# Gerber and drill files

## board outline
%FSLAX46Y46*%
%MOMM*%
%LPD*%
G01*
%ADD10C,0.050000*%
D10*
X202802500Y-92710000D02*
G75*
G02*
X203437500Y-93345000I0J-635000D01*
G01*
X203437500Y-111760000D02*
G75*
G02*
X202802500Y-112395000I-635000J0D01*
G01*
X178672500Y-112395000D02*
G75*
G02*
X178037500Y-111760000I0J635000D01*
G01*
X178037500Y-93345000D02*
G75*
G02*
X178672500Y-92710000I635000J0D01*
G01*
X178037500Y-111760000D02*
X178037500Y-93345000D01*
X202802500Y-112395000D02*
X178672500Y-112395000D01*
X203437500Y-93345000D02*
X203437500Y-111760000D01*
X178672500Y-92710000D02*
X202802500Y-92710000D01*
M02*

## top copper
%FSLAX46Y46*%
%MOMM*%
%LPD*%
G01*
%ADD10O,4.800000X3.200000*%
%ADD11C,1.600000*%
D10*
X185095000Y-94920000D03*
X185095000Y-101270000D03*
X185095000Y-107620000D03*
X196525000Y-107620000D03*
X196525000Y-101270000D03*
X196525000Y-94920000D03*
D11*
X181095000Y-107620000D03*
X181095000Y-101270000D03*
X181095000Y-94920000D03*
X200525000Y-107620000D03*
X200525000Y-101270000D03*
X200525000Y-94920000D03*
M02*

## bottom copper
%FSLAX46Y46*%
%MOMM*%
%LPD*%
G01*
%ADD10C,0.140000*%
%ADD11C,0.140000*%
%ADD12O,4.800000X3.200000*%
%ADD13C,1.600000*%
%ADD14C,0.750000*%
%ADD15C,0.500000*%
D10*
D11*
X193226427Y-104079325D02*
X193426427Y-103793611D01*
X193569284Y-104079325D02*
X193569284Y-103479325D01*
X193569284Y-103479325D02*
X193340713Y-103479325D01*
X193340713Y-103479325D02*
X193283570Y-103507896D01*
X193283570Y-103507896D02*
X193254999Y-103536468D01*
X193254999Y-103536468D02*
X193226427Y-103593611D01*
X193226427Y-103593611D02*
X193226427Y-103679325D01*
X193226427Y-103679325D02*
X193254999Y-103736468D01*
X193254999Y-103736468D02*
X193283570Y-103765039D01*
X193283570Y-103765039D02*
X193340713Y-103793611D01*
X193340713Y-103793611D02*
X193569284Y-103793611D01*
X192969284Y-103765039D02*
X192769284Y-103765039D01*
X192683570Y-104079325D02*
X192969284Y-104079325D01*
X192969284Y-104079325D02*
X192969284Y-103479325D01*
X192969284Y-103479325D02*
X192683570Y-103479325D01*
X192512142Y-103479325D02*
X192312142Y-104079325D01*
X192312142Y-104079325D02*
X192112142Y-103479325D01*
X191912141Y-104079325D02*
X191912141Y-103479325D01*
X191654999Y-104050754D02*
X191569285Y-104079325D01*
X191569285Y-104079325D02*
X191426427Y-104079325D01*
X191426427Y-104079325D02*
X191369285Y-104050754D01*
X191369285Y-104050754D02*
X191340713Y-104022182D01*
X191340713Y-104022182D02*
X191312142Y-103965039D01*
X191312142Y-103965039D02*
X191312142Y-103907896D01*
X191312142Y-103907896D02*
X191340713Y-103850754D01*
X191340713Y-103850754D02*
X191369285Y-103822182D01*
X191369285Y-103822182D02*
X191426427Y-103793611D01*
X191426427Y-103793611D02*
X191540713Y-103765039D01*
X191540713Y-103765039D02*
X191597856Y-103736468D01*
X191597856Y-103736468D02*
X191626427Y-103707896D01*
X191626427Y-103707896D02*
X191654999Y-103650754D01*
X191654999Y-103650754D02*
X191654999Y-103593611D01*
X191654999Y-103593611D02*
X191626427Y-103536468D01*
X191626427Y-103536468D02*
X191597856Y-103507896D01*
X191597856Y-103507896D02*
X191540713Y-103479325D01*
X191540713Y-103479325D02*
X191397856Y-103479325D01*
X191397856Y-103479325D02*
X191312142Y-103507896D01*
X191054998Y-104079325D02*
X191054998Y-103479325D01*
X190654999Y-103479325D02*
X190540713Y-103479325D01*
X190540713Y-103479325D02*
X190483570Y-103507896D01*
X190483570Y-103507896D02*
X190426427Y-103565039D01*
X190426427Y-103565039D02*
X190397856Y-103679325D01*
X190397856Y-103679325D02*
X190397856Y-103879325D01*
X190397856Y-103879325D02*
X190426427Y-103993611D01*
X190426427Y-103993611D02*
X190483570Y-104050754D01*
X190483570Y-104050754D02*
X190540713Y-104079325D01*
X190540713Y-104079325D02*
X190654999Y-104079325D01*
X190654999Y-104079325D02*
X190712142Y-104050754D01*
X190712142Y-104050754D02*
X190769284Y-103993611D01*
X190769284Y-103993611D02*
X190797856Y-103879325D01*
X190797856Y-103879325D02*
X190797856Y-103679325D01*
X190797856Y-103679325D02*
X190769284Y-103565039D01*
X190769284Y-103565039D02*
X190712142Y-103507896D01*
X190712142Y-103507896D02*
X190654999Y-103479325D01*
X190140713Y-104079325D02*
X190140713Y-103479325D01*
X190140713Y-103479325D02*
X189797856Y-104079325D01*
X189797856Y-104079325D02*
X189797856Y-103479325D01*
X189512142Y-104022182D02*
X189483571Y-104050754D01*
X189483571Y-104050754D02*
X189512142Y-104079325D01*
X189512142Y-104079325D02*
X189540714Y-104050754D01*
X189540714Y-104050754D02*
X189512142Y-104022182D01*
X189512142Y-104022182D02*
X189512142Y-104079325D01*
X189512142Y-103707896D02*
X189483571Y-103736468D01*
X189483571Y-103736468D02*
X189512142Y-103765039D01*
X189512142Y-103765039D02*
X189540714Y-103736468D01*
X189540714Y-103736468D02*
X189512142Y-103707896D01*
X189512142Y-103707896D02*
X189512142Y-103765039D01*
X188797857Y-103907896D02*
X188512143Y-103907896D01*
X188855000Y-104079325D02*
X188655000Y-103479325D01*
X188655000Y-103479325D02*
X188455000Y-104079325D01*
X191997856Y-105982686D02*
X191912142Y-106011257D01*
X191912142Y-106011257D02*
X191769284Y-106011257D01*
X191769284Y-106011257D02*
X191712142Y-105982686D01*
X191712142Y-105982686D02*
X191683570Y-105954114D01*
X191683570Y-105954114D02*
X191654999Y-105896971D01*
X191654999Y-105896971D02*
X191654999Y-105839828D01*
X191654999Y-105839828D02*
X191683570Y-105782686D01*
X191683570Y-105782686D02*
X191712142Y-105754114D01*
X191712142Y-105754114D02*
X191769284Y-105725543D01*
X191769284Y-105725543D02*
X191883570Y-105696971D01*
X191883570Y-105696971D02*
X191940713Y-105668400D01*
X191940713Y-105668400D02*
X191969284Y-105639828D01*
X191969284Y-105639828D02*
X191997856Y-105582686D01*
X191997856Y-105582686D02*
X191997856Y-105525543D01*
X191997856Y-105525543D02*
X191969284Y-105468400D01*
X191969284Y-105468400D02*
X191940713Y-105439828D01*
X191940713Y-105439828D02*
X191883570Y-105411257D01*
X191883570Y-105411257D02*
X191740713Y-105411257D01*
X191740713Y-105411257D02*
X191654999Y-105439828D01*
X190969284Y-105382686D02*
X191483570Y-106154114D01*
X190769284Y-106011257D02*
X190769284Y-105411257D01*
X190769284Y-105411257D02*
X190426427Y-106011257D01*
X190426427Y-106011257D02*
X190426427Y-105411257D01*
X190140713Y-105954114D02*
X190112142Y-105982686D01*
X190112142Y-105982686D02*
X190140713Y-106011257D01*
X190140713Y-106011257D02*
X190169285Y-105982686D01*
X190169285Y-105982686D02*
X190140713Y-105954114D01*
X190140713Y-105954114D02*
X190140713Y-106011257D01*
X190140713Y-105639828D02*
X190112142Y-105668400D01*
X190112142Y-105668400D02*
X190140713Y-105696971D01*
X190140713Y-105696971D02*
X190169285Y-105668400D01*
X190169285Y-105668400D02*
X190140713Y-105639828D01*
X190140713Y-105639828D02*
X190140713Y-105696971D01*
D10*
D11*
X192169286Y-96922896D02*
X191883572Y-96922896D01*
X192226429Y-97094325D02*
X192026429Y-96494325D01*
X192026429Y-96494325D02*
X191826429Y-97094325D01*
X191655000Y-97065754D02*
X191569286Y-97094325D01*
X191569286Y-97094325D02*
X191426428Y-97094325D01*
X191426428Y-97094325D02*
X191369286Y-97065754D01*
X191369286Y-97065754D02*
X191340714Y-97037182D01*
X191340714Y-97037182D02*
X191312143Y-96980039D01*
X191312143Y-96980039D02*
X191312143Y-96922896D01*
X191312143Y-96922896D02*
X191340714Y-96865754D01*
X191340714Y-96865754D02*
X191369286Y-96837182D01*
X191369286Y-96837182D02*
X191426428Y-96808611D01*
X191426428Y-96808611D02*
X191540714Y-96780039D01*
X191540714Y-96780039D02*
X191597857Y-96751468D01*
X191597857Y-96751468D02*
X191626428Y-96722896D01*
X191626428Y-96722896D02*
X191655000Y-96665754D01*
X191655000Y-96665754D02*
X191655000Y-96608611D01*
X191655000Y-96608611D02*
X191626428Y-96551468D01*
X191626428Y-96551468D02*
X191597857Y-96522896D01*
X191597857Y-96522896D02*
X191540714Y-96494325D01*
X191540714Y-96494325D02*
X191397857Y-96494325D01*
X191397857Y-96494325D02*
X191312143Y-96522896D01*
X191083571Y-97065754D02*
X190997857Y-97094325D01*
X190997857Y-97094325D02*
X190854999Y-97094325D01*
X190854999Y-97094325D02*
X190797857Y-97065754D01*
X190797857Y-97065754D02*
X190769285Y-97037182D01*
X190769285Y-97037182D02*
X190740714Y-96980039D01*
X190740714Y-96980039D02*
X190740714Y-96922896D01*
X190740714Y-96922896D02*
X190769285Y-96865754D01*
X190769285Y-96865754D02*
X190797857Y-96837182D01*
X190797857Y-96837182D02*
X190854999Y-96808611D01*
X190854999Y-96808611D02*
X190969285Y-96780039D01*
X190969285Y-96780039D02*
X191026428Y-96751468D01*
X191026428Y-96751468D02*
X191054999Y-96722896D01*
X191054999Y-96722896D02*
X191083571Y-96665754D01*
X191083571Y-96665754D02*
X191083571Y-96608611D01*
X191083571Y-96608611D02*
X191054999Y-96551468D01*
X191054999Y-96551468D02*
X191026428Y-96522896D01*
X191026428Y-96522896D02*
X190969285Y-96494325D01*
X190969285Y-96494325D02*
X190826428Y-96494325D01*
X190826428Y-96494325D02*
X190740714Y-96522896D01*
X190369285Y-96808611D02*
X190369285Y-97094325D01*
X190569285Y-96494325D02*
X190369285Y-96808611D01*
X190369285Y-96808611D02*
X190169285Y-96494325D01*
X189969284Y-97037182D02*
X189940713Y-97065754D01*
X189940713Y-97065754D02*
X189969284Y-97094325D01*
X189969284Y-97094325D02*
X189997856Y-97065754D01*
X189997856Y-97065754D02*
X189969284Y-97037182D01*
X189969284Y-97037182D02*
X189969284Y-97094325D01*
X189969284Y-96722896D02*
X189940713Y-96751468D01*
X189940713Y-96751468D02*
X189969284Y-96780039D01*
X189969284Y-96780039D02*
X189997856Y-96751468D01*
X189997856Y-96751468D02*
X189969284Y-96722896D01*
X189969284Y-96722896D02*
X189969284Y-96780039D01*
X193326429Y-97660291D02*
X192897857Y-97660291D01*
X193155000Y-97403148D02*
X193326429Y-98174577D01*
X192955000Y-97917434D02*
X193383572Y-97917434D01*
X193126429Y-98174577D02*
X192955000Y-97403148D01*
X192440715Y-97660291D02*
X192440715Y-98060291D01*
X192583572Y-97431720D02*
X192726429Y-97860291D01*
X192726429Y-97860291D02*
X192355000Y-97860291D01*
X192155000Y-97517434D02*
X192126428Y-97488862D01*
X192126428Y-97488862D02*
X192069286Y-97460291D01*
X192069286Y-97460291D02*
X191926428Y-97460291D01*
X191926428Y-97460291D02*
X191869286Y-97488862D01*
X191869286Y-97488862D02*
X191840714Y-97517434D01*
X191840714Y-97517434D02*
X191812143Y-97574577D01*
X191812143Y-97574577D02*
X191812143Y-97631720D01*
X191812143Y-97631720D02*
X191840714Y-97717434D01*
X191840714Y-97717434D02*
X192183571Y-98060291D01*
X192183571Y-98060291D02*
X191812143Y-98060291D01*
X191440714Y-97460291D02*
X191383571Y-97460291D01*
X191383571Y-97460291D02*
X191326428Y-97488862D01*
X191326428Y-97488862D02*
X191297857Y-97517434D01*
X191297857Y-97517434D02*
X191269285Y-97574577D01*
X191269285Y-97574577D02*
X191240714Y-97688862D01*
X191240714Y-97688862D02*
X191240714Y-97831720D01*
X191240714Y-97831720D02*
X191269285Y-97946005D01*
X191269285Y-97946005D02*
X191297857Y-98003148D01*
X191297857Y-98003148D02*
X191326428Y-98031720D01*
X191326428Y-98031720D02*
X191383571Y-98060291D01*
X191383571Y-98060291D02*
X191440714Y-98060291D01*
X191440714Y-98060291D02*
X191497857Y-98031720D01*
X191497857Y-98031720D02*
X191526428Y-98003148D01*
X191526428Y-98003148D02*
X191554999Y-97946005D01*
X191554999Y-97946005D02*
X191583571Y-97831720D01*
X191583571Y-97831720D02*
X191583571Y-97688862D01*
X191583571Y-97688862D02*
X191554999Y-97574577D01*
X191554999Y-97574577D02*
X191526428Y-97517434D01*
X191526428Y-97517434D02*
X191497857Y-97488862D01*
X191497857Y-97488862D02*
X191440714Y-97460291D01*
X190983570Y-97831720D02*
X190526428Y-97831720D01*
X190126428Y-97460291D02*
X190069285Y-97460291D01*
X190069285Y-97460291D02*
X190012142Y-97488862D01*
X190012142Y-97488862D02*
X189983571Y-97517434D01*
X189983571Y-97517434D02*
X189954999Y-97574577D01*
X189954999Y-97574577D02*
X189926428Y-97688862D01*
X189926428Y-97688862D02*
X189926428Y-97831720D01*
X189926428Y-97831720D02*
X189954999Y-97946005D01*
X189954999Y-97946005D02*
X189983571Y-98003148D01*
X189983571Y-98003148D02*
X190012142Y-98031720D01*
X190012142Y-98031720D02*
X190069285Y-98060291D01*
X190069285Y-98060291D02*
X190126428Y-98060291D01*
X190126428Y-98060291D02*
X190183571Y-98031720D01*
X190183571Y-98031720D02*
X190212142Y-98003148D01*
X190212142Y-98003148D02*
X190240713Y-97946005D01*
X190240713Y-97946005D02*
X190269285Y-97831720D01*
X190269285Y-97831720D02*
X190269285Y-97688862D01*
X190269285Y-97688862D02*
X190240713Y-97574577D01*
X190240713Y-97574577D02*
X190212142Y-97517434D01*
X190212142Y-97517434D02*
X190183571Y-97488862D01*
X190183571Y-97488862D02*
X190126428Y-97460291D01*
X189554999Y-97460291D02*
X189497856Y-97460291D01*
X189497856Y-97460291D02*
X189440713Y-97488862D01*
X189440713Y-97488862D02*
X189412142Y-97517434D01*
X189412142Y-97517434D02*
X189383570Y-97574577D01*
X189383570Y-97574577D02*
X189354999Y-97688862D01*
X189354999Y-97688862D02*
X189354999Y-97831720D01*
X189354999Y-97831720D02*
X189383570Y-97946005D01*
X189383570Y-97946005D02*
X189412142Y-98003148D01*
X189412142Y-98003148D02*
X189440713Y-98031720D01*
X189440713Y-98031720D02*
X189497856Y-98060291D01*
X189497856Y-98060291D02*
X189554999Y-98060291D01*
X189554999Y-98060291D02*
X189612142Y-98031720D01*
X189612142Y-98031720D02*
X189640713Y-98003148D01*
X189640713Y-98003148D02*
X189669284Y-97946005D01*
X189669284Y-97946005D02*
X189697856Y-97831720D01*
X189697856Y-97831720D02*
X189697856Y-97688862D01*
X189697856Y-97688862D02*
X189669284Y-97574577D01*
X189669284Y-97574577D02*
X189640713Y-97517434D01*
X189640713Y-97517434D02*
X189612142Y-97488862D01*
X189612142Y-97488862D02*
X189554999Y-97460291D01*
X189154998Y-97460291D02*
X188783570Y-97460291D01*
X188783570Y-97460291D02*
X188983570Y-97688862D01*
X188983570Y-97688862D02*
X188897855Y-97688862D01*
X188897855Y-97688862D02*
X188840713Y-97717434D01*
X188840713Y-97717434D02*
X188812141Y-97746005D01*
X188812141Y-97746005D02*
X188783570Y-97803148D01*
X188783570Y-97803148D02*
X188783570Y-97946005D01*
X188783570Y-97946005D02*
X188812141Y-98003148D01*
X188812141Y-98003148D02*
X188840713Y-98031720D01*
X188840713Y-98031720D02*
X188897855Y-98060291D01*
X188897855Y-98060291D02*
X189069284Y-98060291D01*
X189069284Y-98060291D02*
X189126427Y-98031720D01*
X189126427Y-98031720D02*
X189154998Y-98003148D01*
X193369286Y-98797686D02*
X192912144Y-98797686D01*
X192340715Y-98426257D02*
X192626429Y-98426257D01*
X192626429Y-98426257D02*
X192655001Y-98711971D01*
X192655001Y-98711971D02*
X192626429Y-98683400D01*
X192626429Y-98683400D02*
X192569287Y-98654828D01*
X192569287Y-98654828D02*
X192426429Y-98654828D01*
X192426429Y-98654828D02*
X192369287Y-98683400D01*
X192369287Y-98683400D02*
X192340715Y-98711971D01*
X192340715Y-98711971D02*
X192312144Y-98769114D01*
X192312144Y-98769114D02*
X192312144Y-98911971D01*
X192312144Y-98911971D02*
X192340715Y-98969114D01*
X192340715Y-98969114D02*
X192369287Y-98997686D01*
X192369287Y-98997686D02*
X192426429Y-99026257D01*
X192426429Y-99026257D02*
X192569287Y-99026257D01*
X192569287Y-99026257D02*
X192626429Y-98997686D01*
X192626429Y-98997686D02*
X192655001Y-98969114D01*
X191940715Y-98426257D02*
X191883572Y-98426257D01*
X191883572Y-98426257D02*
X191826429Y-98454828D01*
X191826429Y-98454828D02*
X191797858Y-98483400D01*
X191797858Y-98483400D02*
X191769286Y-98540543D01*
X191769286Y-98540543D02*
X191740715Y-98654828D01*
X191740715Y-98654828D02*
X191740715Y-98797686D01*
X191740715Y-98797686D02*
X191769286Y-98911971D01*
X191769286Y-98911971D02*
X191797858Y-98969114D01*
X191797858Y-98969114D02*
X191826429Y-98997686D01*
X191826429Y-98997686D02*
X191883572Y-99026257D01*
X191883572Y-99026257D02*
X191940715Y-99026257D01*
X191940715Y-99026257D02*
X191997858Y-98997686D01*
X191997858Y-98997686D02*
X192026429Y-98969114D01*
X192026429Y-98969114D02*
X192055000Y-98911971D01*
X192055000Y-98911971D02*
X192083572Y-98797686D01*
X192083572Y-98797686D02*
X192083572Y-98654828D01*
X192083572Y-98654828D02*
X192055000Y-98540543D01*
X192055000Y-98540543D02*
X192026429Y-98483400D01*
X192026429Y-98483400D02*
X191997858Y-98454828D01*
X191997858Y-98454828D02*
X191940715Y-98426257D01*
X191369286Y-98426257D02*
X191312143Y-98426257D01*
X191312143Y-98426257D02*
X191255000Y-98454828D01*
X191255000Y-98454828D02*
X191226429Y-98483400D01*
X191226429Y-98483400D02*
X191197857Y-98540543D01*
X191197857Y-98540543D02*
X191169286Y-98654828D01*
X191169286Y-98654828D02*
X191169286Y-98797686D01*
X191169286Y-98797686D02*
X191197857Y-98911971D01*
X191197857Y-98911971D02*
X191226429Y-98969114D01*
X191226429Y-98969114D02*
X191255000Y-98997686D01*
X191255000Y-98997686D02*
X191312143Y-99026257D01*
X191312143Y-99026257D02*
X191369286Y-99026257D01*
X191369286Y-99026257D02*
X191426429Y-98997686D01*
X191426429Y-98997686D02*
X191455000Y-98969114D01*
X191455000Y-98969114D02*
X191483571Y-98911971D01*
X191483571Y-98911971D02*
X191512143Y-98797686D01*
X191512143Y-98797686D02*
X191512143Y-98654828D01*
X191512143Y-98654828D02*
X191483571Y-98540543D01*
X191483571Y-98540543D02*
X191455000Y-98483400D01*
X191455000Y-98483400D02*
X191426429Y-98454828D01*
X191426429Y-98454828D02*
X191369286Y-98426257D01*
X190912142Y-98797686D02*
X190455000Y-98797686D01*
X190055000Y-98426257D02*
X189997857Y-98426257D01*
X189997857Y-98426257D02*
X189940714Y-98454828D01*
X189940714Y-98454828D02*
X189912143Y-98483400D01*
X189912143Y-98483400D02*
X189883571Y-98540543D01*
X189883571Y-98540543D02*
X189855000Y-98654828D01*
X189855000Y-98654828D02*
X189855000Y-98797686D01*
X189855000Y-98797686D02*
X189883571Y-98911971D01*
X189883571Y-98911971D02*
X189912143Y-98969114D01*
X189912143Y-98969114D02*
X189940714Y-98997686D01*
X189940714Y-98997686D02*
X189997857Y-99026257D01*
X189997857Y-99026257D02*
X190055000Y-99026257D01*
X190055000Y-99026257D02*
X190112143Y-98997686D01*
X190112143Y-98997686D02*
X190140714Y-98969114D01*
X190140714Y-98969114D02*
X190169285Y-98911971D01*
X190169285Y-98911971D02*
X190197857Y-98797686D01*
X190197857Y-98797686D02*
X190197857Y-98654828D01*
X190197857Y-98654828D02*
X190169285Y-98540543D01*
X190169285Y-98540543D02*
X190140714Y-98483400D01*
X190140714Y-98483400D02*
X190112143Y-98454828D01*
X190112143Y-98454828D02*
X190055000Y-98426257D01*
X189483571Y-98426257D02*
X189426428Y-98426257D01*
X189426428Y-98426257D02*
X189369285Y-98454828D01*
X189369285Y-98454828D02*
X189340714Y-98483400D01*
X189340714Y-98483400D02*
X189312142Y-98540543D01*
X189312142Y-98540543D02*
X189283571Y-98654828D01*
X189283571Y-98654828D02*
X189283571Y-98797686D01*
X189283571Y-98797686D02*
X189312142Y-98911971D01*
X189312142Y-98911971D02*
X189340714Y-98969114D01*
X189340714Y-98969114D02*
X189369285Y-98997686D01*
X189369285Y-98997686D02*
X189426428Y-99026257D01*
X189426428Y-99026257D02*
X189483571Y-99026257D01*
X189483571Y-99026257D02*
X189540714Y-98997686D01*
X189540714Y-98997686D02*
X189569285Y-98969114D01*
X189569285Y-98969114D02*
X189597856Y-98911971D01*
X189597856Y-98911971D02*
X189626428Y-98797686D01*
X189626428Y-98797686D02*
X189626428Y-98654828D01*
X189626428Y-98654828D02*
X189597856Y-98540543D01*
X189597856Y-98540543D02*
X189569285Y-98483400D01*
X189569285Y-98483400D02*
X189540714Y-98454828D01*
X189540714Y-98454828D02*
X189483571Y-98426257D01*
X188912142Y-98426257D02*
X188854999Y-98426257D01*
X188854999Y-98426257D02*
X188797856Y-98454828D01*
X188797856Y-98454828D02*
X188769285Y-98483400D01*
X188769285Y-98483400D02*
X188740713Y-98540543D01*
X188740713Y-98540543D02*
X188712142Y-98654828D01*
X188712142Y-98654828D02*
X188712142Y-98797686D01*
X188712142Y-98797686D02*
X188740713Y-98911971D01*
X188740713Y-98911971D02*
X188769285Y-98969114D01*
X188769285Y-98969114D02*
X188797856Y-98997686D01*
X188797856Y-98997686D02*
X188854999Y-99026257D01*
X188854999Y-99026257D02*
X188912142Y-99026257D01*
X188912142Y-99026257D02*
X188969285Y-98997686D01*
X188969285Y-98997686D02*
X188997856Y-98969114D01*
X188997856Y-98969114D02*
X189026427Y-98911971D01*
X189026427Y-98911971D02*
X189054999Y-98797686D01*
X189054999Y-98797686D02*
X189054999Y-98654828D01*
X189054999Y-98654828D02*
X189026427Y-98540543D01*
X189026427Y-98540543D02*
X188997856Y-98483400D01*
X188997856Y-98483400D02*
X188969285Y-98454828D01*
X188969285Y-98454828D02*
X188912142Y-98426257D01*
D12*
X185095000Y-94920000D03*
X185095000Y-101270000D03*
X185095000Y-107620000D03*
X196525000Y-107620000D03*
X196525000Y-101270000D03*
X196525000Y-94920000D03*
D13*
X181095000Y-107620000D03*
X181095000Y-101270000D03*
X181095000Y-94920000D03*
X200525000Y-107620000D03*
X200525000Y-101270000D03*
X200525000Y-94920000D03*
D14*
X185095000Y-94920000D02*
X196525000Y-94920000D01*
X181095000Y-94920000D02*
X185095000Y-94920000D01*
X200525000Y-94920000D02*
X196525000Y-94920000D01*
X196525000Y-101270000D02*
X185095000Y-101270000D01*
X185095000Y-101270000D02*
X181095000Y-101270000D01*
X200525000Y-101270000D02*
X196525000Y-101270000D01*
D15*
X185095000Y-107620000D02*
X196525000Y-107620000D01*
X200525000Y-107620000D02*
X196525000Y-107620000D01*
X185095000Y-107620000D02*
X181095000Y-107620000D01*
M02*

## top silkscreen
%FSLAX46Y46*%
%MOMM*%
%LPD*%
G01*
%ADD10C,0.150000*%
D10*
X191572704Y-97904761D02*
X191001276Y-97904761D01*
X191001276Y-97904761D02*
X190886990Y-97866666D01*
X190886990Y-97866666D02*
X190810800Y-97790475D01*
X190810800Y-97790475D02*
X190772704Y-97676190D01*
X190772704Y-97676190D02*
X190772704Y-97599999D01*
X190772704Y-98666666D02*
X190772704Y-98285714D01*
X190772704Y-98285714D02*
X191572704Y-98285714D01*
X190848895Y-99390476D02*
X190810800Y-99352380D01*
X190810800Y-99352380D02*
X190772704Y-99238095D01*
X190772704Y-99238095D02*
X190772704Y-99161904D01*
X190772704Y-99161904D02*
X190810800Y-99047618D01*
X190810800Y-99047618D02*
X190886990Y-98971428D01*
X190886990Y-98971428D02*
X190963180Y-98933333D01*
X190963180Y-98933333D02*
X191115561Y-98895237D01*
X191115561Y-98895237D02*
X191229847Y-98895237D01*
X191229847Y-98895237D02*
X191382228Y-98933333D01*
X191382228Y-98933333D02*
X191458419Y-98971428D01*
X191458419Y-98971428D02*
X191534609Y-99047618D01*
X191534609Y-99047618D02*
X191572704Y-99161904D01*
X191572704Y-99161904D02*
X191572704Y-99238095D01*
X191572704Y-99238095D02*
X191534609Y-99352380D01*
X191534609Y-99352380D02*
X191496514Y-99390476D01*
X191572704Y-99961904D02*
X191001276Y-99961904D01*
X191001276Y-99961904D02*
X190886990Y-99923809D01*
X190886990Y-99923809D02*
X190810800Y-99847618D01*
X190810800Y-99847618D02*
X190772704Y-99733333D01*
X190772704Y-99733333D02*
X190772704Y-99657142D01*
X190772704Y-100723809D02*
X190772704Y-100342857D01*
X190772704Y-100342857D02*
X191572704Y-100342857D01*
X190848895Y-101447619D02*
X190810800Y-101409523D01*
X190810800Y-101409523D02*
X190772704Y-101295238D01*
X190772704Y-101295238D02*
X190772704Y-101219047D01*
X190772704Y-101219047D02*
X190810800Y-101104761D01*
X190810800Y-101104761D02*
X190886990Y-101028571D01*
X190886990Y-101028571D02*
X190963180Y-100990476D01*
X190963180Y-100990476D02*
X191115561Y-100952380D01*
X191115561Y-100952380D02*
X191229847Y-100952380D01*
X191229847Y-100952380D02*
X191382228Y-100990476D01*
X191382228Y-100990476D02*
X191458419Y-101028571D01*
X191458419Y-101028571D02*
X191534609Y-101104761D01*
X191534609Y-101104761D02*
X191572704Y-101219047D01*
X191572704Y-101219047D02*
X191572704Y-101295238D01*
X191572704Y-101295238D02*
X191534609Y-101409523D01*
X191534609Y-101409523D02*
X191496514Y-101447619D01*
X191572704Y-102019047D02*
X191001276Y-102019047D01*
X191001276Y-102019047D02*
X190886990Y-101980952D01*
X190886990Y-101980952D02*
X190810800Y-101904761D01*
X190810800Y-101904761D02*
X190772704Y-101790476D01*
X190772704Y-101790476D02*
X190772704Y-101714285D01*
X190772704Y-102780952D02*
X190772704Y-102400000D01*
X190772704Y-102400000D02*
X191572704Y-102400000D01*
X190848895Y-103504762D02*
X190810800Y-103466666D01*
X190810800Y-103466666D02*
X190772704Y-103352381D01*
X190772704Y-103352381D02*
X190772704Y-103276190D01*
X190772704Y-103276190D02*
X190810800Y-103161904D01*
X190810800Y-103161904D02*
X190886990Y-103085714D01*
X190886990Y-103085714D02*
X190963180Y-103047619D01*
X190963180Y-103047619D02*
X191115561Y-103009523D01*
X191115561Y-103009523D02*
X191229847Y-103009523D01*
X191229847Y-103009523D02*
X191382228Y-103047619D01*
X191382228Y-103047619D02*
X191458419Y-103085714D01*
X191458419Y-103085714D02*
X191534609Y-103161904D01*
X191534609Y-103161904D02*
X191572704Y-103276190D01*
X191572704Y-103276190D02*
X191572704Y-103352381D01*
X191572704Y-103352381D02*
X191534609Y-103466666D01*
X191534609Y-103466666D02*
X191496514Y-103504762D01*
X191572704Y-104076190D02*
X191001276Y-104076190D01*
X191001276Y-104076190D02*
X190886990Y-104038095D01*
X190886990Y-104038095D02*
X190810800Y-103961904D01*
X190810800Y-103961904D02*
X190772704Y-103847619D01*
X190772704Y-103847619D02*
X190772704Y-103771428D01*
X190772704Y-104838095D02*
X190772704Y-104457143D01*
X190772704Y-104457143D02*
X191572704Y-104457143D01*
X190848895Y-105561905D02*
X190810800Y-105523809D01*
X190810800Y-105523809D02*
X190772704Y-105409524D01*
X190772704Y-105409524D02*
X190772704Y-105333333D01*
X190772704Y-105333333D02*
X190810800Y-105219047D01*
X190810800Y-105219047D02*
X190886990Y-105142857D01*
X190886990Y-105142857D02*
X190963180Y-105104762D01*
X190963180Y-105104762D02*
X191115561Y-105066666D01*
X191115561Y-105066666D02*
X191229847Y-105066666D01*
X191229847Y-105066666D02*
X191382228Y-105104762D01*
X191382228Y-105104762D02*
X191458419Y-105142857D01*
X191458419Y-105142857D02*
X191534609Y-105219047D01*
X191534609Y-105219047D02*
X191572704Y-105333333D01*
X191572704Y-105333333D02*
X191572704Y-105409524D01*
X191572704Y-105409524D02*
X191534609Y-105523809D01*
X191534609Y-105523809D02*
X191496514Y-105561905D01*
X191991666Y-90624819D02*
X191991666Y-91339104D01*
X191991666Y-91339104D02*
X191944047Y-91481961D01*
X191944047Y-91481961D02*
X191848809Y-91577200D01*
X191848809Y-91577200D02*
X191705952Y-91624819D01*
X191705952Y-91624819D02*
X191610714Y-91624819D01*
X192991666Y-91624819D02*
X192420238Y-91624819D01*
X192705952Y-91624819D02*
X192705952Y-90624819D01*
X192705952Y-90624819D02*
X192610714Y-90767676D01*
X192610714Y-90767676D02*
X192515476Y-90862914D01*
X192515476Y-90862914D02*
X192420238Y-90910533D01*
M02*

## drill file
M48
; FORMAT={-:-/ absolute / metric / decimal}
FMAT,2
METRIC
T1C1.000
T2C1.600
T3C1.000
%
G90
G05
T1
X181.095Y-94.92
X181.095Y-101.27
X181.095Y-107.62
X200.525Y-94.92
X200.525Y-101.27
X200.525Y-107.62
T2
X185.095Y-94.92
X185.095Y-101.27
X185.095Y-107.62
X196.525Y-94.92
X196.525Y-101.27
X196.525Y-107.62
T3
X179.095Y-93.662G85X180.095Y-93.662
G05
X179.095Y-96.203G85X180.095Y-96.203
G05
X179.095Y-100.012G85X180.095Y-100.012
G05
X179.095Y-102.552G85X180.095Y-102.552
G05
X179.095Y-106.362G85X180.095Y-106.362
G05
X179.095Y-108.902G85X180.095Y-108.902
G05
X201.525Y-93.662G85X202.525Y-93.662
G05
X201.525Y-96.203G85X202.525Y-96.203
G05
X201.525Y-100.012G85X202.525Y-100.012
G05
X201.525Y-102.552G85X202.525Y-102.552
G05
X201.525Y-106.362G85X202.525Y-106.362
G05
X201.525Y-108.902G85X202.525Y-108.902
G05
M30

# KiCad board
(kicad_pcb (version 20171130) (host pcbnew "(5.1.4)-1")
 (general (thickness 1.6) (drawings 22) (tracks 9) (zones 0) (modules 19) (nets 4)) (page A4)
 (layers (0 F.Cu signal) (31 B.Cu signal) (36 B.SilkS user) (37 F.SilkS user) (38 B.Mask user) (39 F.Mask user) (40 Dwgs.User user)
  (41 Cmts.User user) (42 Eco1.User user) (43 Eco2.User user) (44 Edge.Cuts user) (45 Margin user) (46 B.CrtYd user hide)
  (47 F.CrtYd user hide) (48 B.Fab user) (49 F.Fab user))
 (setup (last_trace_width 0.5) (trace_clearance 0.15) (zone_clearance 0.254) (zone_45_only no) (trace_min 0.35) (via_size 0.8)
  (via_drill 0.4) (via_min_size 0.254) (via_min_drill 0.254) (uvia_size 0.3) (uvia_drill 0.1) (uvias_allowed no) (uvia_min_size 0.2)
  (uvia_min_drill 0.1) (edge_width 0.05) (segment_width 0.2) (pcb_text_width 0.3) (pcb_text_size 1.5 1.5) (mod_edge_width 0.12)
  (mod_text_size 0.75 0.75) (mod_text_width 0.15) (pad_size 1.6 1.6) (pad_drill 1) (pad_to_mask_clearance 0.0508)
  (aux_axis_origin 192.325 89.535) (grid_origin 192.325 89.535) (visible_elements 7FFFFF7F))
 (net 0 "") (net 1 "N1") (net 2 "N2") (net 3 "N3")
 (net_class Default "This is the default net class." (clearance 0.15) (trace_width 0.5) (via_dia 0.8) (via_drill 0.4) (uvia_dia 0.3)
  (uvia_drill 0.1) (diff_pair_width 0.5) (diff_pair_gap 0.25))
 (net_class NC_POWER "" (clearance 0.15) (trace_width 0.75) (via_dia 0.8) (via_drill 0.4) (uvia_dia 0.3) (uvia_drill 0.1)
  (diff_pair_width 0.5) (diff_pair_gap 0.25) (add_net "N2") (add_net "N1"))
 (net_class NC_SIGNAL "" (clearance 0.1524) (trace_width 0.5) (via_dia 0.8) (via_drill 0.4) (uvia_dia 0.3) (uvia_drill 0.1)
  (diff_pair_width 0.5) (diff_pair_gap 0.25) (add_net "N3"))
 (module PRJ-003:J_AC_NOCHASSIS (layer F.Cu) (at 192.325 90.17)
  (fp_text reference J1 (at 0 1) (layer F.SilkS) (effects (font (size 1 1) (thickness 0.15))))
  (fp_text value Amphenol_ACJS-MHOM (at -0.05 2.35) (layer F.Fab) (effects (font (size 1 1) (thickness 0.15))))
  (pad "" connect circle (at 4.2 4.75) (size 1.6 1.6) (layers F.Mask))
  (pad "" connect circle (at 4.2 11.1) (size 1.6 1.6) (layers F.Mask))
  (pad "" connect circle (at 4.2 17.45) (size 1.6 1.6) (layers F.Mask))
  (pad "" connect circle (at -7.23 17.45) (size 1.6 1.6) (layers F.Mask))
  (pad "" connect circle (at -7.23 11.1) (size 1.6 1.6) (layers F.Mask))
  (pad "" connect circle (at -7.23 4.75) (size 1.6 1.6) (layers F.Mask))
  (pad S thru_hole oval (at -7.23 4.75) (size 4.8 3.2) (drill 1.6) (layers B.Cu B.Mask) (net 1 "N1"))
  (pad R thru_hole oval (at -7.23 11.1) (size 4.8 3.2) (drill 1.6) (layers B.Cu B.Mask) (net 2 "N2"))
  (pad T thru_hole oval (at -7.23 17.45) (size 4.8 3.2) (drill 1.6) (layers B.Cu B.Mask) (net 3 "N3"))
  (pad TN thru_hole oval (at 4.2 17.45) (size 4.8 3.2) (drill 1.6) (layers B.Cu B.Mask) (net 3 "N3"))
  (pad RN thru_hole oval (at 4.2 11.1) (size 4.8 3.2) (drill 1.6) (layers B.Cu B.Mask) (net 2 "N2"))
  (pad SN thru_hole oval (at 4.2 4.75) (size 4.8 3.2) (drill 1.6) (layers B.Cu B.Mask) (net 1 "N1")))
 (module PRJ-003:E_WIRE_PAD (layer F.Cu) (at 181.095 107.62)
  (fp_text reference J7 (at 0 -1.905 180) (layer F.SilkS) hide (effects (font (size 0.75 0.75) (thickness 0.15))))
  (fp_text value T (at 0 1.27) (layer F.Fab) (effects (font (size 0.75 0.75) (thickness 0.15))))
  (pad "" connect circle (at 0 0) (size 1 1) (layers F.Mask))
  (pad 1 thru_hole circle (at 0 0) (size 1.6 1.6) (drill 1) (layers B.Cu B.Mask) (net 3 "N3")))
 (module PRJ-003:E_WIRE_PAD (layer F.Cu) (at 181.095 101.27)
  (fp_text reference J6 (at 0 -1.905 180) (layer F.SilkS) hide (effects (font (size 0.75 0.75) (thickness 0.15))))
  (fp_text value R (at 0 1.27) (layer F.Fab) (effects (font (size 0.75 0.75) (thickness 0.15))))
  (pad "" connect circle (at 0 0) (size 1 1) (layers F.Mask))
  (pad 1 thru_hole circle (at 0 0) (size 1.6 1.6) (drill 1) (layers B.Cu B.Mask) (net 2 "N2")))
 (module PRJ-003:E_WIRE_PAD (layer F.Cu) (at 181.095 94.92)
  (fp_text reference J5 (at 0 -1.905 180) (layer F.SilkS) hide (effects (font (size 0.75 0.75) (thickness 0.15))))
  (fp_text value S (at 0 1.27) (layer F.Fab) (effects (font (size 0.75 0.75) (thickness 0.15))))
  (pad "" connect circle (at 0 0) (size 1 1) (layers F.Mask))
  (pad 1 thru_hole circle (at 0 0) (size 1.6 1.6) (drill 1) (layers B.Cu B.Mask) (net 1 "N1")))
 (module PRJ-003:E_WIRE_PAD (layer F.Cu) (at 200.525 107.62)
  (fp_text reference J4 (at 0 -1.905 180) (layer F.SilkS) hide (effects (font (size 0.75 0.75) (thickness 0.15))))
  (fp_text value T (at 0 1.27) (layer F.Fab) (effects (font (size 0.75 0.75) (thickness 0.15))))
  (pad "" connect circle (at 0 0) (size 1 1) (layers F.Mask))
  (pad 1 thru_hole circle (at 0 0) (size 1.6 1.6) (drill 1) (layers B.Cu B.Mask) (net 3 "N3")))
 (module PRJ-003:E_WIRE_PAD (layer F.Cu) (at 200.525 101.27)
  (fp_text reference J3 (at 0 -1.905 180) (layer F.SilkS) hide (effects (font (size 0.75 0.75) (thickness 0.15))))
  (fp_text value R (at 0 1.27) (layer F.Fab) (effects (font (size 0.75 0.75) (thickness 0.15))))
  (pad "" connect circle (at 0 0) (size 1 1) (layers F.Mask))
  (pad 1 thru_hole circle (at 0 0) (size 1.6 1.6) (drill 1) (layers B.Cu B.Mask) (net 2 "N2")))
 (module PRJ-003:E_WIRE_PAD (layer F.Cu) (at 200.525 94.92)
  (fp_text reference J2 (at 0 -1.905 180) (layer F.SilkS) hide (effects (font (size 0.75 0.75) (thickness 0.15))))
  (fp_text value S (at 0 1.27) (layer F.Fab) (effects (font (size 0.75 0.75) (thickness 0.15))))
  (pad "" connect circle (at 0 0) (size 1 1) (layers F.Mask))
  (pad 1 thru_hole circle (at 0 0) (size 1.6 1.6) (drill 1) (layers B.Cu B.Mask) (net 1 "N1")))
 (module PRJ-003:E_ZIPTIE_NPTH (layer F.Cu) (at 202.025 108.9025 90)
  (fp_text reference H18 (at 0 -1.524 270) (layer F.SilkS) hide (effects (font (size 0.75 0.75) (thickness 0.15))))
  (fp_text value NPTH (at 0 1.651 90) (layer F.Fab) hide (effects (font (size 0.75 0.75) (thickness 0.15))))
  (pad "" np_thru_hole oval (at 0 0 90) (size 1 2) (drill oval 1 2) (layers *.Cu *.Mask)))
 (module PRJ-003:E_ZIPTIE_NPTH (layer F.Cu) (at 202.025 102.5525 90)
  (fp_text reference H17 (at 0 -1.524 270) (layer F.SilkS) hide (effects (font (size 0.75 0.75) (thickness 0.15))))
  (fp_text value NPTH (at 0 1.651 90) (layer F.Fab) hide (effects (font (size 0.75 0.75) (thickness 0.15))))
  (pad "" np_thru_hole oval (at 0 0 90) (size 1 2) (drill oval 1 2) (layers *.Cu *.Mask)))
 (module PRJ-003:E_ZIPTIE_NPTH (layer F.Cu) (at 202.025 106.3625 90)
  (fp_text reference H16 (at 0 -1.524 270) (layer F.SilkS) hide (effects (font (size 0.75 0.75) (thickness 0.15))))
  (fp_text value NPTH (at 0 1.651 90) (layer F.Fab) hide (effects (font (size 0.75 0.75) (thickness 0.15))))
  (pad "" np_thru_hole oval (at 0 0 90) (size 1 2) (drill oval 1 2) (layers *.Cu *.Mask)))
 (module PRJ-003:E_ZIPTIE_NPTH (layer F.Cu) (at 202.025 96.2025 90)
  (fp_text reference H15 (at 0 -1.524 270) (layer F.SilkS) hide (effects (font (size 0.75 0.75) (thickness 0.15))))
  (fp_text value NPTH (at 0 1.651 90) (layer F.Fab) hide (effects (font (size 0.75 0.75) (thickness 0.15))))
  (pad "" np_thru_hole oval (at 0 0 90) (size 1 2) (drill oval 1 2) (layers *.Cu *.Mask)))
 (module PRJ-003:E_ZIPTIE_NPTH (layer F.Cu) (at 202.025 100.0125 90)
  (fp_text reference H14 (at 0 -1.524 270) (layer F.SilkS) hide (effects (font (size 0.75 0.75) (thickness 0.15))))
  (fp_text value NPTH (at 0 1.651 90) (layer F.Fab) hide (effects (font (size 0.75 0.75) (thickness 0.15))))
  (pad "" np_thru_hole oval (at 0 0 90) (size 1 2) (drill oval 1 2) (layers *.Cu *.Mask)))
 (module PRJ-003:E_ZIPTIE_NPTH (layer F.Cu) (at 202.025 93.6625 90)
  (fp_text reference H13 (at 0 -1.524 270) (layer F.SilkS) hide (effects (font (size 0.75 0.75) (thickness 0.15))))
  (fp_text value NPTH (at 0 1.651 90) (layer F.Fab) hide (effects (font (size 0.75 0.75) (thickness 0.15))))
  (pad "" np_thru_hole oval (at 0 0 90) (size 1 2) (drill oval 1 2) (layers *.Cu *.Mask)))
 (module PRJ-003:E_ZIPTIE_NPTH (layer F.Cu) (at 179.595 93.6625 90)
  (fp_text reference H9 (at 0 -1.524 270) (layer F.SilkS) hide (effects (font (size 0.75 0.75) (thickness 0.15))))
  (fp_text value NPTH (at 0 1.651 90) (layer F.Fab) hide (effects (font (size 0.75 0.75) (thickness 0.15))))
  (pad "" np_thru_hole oval (at 0 0 90) (size 1 2) (drill oval 1 2) (layers *.Cu *.Mask)))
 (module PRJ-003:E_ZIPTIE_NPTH (layer F.Cu) (at 179.595 96.2025 90)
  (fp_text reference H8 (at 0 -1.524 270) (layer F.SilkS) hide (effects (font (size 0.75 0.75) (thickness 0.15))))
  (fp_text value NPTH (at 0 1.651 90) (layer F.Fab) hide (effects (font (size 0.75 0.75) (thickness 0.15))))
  (pad "" np_thru_hole oval (at 0 0 90) (size 1 2) (drill oval 1 2) (layers *.Cu *.Mask)))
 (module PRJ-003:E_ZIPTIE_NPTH (layer F.Cu) (at 179.595 100.0125 90)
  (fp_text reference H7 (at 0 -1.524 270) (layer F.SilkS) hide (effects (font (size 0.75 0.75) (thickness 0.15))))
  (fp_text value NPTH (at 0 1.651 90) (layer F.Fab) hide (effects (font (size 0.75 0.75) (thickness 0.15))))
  (pad "" np_thru_hole oval (at 0 0 90) (size 1 2) (drill oval 1 2) (layers *.Cu *.Mask)))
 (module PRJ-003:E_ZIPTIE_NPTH (layer F.Cu) (at 179.595 102.5525 90)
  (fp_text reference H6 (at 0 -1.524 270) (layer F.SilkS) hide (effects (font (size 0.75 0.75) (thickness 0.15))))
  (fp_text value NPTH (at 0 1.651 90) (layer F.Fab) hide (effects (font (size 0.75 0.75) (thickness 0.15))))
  (pad "" np_thru_hole oval (at 0 0 90) (size 1 2) (drill oval 1 2) (layers *.Cu *.Mask)))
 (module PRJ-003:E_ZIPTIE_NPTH (layer F.Cu) (at 179.595 106.3625 90)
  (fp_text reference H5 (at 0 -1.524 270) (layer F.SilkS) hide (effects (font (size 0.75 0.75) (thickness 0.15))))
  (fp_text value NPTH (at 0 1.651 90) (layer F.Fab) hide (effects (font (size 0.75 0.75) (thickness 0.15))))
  (pad "" np_thru_hole oval (at 0 0 90) (size 1 2) (drill oval 1 2) (layers *.Cu *.Mask)))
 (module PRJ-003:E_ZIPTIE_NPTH (layer F.Cu) (at 179.595 108.9025 90)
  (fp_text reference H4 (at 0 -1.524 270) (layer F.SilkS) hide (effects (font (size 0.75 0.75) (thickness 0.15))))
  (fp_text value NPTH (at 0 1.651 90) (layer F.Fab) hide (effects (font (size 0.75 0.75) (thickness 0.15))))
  (pad "" np_thru_hole oval (at 0 0 90) (size 1 2) (drill oval 1 2) (layers *.Cu *.Mask)))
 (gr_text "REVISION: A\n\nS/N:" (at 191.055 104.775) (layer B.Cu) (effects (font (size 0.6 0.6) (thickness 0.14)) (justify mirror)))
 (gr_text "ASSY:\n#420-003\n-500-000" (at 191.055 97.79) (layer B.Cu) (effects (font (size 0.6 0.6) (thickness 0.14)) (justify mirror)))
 (gr_arc (start 202.8025 93.345) (end 203.4375 93.345) (angle -90) (layer Edge.Cuts) (width 0.05))
 (gr_arc (start 202.8025 111.76) (end 202.8025 112.395) (angle -90) (layer Edge.Cuts) (width 0.05))
 (gr_arc (start 178.6725 111.76) (end 178.0375 111.76) (angle -90) (layer Edge.Cuts) (width 0.05))
 (gr_arc (start 178.6725 93.345) (end 178.6725 92.71) (angle -90) (layer Edge.Cuts) (width 0.05))
 (gr_line (start 178.0375 111.76) (end 178.0375 93.345) (layer Edge.Cuts) (width 0.05))
 (gr_line (start 202.8025 112.395) (end 178.6725 112.395) (layer Edge.Cuts) (width 0.05))
 (gr_line (start 203.4375 93.345) (end 203.4375 111.76) (layer Edge.Cuts) (width 0.05))
 (gr_line (start 178.6725 92.71) (end 202.8025 92.71) (layer Edge.Cuts) (width 0.05))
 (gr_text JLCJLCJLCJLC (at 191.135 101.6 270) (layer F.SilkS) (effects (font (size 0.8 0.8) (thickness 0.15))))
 (segment (start 185.095 94.92) (end 196.525 94.92) (width 0.75) (layer B.Cu) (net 1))
 (segment (start 181.095 94.92) (end 185.095 94.92) (width 0.75) (layer B.Cu) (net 1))
 (segment (start 200.525 94.92) (end 196.525 94.92) (width 0.75) (layer B.Cu) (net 1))
 (segment (start 196.525 101.27) (end 185.095 101.27) (width 0.75) (layer B.Cu) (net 2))
 (segment (start 185.095 101.27) (end 181.095 101.27) (width 0.75) (layer B.Cu) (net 2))
 (segment (start 200.525 101.27) (end 196.525 101.27) (width 0.75) (layer B.Cu) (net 2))
 (segment (start 185.095 107.62) (end 196.525 107.62) (width 0.5) (layer B.Cu) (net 3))
 (segment (start 200.525 107.62) (end 196.525 107.62) (width 0.5) (layer B.Cu) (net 3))
 (segment (start 185.095 107.62) (end 181.095 107.62) (width 0.5) (layer B.Cu) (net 3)))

